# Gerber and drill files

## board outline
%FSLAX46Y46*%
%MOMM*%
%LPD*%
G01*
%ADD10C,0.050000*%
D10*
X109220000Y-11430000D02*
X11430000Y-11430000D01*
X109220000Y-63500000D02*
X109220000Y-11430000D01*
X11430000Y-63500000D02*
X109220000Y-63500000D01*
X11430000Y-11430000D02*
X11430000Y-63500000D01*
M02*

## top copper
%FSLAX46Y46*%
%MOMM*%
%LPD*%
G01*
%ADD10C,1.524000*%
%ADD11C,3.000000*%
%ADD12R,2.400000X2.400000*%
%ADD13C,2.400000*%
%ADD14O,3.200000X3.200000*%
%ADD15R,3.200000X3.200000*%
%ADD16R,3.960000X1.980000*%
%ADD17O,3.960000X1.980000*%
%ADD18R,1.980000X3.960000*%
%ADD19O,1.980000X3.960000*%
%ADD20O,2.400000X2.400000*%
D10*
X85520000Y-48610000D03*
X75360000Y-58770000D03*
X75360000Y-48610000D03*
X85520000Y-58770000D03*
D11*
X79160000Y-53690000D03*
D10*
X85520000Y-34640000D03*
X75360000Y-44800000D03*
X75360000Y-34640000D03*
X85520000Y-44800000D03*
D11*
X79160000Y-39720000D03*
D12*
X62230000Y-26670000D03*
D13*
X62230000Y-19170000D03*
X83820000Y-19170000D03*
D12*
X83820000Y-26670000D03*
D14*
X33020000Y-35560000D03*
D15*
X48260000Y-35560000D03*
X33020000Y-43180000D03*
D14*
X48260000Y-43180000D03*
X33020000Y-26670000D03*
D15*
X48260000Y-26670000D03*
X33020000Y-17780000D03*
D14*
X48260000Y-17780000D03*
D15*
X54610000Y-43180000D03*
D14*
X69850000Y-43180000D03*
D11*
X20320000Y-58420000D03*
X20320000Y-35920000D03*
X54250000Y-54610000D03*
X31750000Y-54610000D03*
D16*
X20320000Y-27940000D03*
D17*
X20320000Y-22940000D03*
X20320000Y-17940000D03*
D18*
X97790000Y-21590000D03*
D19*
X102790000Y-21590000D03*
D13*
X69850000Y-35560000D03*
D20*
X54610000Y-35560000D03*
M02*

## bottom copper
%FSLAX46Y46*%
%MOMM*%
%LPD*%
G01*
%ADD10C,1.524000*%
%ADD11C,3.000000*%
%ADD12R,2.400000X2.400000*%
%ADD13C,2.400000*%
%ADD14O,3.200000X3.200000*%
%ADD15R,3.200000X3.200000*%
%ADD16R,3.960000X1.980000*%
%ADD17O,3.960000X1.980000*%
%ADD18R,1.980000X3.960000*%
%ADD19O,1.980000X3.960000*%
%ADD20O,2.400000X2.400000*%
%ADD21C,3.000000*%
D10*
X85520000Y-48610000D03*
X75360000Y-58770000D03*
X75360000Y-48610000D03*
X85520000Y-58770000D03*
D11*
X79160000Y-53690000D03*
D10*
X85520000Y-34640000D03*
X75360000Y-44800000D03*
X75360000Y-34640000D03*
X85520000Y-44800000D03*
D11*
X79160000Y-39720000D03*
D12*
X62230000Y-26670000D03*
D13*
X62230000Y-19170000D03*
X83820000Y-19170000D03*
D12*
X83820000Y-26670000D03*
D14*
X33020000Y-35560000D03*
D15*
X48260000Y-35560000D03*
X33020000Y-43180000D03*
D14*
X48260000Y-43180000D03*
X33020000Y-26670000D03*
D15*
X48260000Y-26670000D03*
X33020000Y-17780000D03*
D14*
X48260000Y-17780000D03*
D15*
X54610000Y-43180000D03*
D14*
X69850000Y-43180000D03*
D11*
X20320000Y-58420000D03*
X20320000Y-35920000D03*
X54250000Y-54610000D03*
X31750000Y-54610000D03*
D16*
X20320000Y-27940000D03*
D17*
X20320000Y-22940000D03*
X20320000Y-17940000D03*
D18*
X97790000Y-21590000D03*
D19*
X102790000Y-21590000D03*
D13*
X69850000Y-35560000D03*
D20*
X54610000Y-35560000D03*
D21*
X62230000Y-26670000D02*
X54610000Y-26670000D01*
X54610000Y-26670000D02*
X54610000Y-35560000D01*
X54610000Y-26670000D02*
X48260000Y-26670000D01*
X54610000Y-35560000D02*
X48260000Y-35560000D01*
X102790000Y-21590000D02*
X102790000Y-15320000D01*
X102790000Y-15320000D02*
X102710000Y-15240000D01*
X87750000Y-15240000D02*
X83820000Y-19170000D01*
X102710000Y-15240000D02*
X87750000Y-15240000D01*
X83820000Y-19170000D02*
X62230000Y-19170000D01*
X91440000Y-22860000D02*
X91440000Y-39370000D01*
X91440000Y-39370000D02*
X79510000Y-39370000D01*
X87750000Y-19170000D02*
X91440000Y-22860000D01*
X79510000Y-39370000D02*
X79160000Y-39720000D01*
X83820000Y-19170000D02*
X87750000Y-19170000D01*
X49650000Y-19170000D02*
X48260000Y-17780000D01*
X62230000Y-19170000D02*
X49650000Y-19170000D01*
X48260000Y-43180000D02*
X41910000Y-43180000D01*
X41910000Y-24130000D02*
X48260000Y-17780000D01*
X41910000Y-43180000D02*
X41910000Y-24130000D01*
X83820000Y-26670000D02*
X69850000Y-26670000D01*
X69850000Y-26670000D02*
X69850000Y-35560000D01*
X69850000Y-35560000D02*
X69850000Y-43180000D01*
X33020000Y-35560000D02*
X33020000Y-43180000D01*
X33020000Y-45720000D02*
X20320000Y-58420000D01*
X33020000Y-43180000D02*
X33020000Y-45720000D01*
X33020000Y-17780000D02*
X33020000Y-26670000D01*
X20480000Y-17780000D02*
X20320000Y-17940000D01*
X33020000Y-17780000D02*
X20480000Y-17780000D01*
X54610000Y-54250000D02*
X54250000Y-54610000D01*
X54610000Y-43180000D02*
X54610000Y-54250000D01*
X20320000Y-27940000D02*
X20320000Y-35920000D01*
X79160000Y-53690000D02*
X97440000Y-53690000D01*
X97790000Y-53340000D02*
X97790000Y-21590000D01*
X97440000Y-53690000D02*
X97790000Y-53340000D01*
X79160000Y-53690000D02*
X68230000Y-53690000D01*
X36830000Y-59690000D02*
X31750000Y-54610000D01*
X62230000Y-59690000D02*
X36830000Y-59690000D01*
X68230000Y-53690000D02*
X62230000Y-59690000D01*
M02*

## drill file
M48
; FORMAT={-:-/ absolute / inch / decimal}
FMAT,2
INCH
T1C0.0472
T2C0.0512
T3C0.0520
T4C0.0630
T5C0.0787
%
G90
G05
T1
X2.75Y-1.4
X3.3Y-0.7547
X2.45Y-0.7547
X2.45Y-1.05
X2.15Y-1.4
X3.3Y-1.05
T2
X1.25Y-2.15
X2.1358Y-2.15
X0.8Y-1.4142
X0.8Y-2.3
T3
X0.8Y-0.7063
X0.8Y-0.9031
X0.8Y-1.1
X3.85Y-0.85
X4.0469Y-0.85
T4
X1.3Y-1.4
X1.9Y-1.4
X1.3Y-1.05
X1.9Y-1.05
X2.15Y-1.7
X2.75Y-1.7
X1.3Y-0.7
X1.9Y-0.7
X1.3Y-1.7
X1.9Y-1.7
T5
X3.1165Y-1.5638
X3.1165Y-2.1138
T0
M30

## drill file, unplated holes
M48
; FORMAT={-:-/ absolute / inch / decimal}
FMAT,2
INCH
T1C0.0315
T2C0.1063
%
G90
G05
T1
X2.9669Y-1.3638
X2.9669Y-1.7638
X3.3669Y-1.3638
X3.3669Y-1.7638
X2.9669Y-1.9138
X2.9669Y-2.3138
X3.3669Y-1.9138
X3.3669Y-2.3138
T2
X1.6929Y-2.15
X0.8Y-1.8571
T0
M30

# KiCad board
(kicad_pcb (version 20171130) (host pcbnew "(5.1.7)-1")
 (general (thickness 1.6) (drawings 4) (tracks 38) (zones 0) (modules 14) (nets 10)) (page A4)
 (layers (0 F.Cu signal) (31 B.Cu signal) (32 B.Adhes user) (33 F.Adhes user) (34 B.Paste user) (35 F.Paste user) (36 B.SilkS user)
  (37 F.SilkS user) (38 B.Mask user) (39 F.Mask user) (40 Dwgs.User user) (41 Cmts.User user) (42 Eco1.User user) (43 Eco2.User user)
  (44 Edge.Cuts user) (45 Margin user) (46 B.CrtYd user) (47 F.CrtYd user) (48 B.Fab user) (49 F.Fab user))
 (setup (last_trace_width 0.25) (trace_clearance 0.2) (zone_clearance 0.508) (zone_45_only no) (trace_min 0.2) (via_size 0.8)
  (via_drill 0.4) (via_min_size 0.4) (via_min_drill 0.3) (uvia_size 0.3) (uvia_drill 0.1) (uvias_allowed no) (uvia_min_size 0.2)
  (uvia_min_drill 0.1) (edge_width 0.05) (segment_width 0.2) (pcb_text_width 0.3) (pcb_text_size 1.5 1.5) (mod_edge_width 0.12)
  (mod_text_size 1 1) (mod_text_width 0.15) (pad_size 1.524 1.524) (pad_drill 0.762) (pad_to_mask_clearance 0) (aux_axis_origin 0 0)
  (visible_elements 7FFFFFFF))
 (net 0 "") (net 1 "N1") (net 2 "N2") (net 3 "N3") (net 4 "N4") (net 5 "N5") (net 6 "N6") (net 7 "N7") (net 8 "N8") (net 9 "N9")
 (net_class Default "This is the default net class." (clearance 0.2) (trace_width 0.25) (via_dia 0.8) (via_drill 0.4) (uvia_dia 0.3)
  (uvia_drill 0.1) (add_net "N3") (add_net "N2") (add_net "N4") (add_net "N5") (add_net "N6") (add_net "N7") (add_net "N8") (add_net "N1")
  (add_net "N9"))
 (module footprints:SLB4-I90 (layer F.Cu) (at 73.66 59.69)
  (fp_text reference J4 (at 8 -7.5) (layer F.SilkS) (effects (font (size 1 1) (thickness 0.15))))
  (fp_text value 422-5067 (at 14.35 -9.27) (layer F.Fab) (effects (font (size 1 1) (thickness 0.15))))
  (pad "" np_thru_hole circle (at 11.86 -11.08) (size 1.524 1.524) (drill 0.8) (layers *.Cu *.Mask))
  (pad "" np_thru_hole circle (at 1.7 -0.92) (size 1.524 1.524) (drill 0.8) (layers *.Cu *.Mask))
  (pad "" np_thru_hole circle (at 1.7 -11.08) (size 1.524 1.524) (drill 0.8) (layers *.Cu *.Mask))
  (pad "" np_thru_hole circle (at 11.86 -0.92) (size 1.524 1.524) (drill 0.8) (layers *.Cu *.Mask))
  (pad 1 thru_hole circle (at 5.5 -6) (size 3 3) (drill 2) (layers *.Cu *.Mask) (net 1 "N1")))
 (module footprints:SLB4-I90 (layer F.Cu) (at 73.66 45.72)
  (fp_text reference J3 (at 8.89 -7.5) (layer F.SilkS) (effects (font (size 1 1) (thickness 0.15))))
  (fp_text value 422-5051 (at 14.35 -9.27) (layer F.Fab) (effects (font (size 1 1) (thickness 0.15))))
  (pad "" np_thru_hole circle (at 11.86 -11.08) (size 1.524 1.524) (drill 0.8) (layers *.Cu *.Mask))
  (pad "" np_thru_hole circle (at 1.7 -0.92) (size 1.524 1.524) (drill 0.8) (layers *.Cu *.Mask))
  (pad "" np_thru_hole circle (at 1.7 -11.08) (size 1.524 1.524) (drill 0.8) (layers *.Cu *.Mask))
  (pad "" np_thru_hole circle (at 11.86 -0.92) (size 1.524 1.524) (drill 0.8) (layers *.Cu *.Mask))
  (pad 1 thru_hole circle (at 5.5 -6) (size 3 3) (drill 2) (layers *.Cu *.Mask) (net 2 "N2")))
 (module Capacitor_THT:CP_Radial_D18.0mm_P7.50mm (layer F.Cu) (at 62.23 26.67 90)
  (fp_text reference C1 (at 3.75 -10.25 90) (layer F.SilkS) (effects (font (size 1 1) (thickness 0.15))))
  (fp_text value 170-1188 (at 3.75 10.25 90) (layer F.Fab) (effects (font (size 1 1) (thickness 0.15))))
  (pad 1 thru_hole rect (at 0 0 90) (size 2.4 2.4) (drill 1.2) (layers *.Cu *.Mask) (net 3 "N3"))
  (pad 2 thru_hole circle (at 7.5 0 90) (size 2.4 2.4) (drill 1.2) (layers *.Cu *.Mask) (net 2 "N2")))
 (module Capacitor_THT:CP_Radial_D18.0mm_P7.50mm (layer F.Cu) (at 83.82 26.67 90)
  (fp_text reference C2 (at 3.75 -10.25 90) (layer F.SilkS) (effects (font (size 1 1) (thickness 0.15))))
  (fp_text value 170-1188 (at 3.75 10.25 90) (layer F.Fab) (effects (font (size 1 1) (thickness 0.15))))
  (pad 2 thru_hole circle (at 7.5 0 90) (size 2.4 2.4) (drill 1.2) (layers *.Cu *.Mask) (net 2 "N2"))
  (pad 1 thru_hole rect (at 0 0 90) (size 2.4 2.4) (drill 1.2) (layers *.Cu *.Mask) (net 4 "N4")))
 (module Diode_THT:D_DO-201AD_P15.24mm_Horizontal (layer F.Cu) (at 48.26 35.56 180)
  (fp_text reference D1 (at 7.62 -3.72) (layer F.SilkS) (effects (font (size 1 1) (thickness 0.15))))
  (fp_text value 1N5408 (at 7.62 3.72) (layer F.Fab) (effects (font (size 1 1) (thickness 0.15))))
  (pad 2 thru_hole oval (at 15.24 0 180) (size 3.2 3.2) (drill 1.6) (layers *.Cu *.Mask) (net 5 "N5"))
  (pad 1 thru_hole rect (at 0 0 180) (size 3.2 3.2) (drill 1.6) (layers *.Cu *.Mask) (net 3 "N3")))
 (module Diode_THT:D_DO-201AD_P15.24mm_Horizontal (layer F.Cu) (at 33.02 43.18)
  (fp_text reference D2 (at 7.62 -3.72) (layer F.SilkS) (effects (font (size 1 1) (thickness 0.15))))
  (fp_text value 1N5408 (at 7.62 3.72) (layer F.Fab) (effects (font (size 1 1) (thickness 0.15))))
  (pad 1 thru_hole rect (at 0 0) (size 3.2 3.2) (drill 1.6) (layers *.Cu *.Mask) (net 5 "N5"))
  (pad 2 thru_hole oval (at 15.24 0) (size 3.2 3.2) (drill 1.6) (layers *.Cu *.Mask) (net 2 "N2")))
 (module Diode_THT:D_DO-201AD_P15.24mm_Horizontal (layer F.Cu) (at 48.26 26.67 180)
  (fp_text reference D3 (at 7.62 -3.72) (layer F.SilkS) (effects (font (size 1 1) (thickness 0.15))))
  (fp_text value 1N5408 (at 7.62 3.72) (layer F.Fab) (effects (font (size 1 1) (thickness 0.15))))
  (pad 2 thru_hole oval (at 15.24 0 180) (size 3.2 3.2) (drill 1.6) (layers *.Cu *.Mask) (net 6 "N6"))
  (pad 1 thru_hole rect (at 0 0 180) (size 3.2 3.2) (drill 1.6) (layers *.Cu *.Mask) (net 3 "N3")))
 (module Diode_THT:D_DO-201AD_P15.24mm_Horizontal (layer F.Cu) (at 33.02 17.78)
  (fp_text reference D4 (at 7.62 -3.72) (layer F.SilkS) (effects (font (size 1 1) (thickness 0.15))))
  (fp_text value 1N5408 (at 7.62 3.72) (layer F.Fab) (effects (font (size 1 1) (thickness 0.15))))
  (pad 1 thru_hole rect (at 0 0) (size 3.2 3.2) (drill 1.6) (layers *.Cu *.Mask) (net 6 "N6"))
  (pad 2 thru_hole oval (at 15.24 0) (size 3.2 3.2) (drill 1.6) (layers *.Cu *.Mask) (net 2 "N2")))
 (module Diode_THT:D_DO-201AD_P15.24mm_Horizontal (layer F.Cu) (at 54.61 43.18)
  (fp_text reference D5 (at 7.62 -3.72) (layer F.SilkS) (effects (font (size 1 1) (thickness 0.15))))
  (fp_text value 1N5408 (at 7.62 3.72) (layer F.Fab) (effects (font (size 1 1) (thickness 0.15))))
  (pad 1 thru_hole rect (at 0 0) (size 3.2 3.2) (drill 1.6) (layers *.Cu *.Mask) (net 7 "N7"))
  (pad 2 thru_hole oval (at 15.24 0) (size 3.2 3.2) (drill 1.6) (layers *.Cu *.Mask) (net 4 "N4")))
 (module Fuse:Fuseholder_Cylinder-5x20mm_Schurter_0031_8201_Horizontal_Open (layer F.Cu) (at 20.32 58.42 90)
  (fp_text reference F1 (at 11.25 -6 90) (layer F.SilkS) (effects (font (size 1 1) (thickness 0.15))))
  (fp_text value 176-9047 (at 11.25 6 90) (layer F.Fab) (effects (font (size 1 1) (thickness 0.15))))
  (pad 1 thru_hole circle (at 0 0 90) (size 3 3) (drill 1.3) (layers *.Cu *.Mask) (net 5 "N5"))
  (pad 2 thru_hole circle (at 22.5 0 90) (size 3 3) (drill 1.3) (layers *.Cu *.Mask) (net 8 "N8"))
  (pad "" np_thru_hole circle (at 11.25 0 90) (size 2.7 2.7) (drill 2.7) (layers *.Cu *.Mask)))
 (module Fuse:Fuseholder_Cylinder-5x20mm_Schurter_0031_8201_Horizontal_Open (layer F.Cu) (at 31.75 54.61)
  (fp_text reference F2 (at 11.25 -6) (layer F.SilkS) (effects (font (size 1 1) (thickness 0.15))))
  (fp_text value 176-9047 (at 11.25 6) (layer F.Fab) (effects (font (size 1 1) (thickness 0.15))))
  (pad "" np_thru_hole circle (at 11.25 0) (size 2.7 2.7) (drill 2.7) (layers *.Cu *.Mask))
  (pad 2 thru_hole circle (at 22.5 0) (size 3 3) (drill 1.3) (layers *.Cu *.Mask) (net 7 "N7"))
  (pad 1 thru_hole circle (at 0 0) (size 3 3) (drill 1.3) (layers *.Cu *.Mask) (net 1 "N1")))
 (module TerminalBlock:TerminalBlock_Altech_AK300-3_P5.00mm (layer F.Cu) (at 20.32 27.94 90)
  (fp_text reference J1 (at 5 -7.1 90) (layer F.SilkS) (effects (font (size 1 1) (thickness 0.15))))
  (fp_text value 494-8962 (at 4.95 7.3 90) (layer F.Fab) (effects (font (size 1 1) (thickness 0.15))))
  (pad 1 thru_hole rect (at 0 0 90) (size 1.98 3.96) (drill 1.32) (layers *.Cu *.Mask) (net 8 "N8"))
  (pad 2 thru_hole oval (at 5 0 90) (size 1.98 3.96) (drill 1.32) (layers *.Cu *.Mask) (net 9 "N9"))
  (pad 3 thru_hole oval (at 10 0 90) (size 1.98 3.96) (drill 1.32) (layers *.Cu *.Mask) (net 6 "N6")))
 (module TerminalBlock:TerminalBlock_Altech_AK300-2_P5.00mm (layer F.Cu) (at 97.79 21.59)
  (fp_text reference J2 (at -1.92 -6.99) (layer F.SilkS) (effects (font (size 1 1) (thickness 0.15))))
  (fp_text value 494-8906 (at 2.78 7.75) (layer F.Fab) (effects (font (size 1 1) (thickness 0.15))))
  (pad 1 thru_hole rect (at 0 0) (size 1.98 3.96) (drill 1.32) (layers *.Cu *.Mask) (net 1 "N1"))
  (pad 2 thru_hole oval (at 5 0) (size 1.98 3.96) (drill 1.32) (layers *.Cu *.Mask) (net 2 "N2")))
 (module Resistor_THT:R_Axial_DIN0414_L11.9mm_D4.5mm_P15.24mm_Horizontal (layer F.Cu) (at 69.85 35.56 180)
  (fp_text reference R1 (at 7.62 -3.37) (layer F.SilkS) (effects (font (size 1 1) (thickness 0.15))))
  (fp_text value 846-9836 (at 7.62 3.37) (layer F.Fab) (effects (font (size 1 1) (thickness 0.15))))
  (pad 1 thru_hole circle (at 0 0 180) (size 2.4 2.4) (drill 1.2) (layers *.Cu *.Mask) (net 4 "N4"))
  (pad 2 thru_hole oval (at 15.24 0 180) (size 2.4 2.4) (drill 1.2) (layers *.Cu *.Mask) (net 3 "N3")))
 (gr_line (start 109.22 11.43) (end 11.43 11.43) (layer Edge.Cuts) (width 0.05))
 (gr_line (start 109.22 63.5) (end 109.22 11.43) (layer Edge.Cuts) (width 0.05))
 (gr_line (start 11.43 63.5) (end 109.22 63.5) (layer Edge.Cuts) (width 0.05))
 (gr_line (start 11.43 11.43) (end 11.43 63.5) (layer Edge.Cuts) (width 0.05))
 (segment (start 62.23 26.67) (end 54.61 26.67) (width 3) (layer B.Cu) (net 3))
 (segment (start 54.61 26.67) (end 54.61 35.56) (width 3) (layer B.Cu) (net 3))
 (segment (start 54.61 26.67) (end 48.26 26.67) (width 3) (layer B.Cu) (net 3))
 (segment (start 54.61 35.56) (end 48.26 35.56) (width 3) (layer B.Cu) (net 3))
 (segment (start 102.79 21.59) (end 102.79 15.32) (width 3) (layer B.Cu) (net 2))
 (segment (start 102.79 15.32) (end 102.71 15.24) (width 3) (layer B.Cu) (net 2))
 (segment (start 87.75 15.24) (end 83.82 19.17) (width 3) (layer B.Cu) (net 2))
 (segment (start 102.71 15.24) (end 87.75 15.24) (width 3) (layer B.Cu) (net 2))
 (segment (start 83.82 19.17) (end 62.23 19.17) (width 3) (layer B.Cu) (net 2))
 (segment (start 91.44 22.86) (end 91.44 39.37) (width 3) (layer B.Cu) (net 2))
 (segment (start 91.44 39.37) (end 79.51 39.37) (width 3) (layer B.Cu) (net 2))
 (segment (start 87.75 19.17) (end 91.44 22.86) (width 3) (layer B.Cu) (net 2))
 (segment (start 79.51 39.37) (end 79.16 39.72) (width 3) (layer B.Cu) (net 2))
 (segment (start 83.82 19.17) (end 87.75 19.17) (width 3) (layer B.Cu) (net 2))
 (segment (start 49.65 19.17) (end 48.26 17.78) (width 3) (layer B.Cu) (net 2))
 (segment (start 62.23 19.17) (end 49.65 19.17) (width 3) (layer B.Cu) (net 2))
 (segment (start 48.26 43.18) (end 41.91 43.18) (width 3) (layer B.Cu) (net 2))
 (segment (start 41.91 24.13) (end 48.26 17.78) (width 3) (layer B.Cu) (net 2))
 (segment (start 41.91 43.18) (end 41.91 24.13) (width 3) (layer B.Cu) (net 2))
 (segment (start 83.82 26.67) (end 69.85 26.67) (width 3) (layer B.Cu) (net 4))
 (segment (start 69.85 26.67) (end 69.85 35.56) (width 3) (layer B.Cu) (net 4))
 (segment (start 69.85 35.56) (end 69.85 43.18) (width 3) (layer B.Cu) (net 4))
 (segment (start 33.02 35.56) (end 33.02 43.18) (width 3) (layer B.Cu) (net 5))
 (segment (start 33.02 45.72) (end 20.32 58.42) (width 3) (layer B.Cu) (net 5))
 (segment (start 33.02 43.18) (end 33.02 45.72) (width 3) (layer B.Cu) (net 5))
 (segment (start 33.02 17.78) (end 33.02 26.67) (width 3) (layer B.Cu) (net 6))
 (segment (start 20.48 17.78) (end 20.32 17.94) (width 3) (layer B.Cu) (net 6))
 (segment (start 33.02 17.78) (end 20.48 17.78) (width 3) (layer B.Cu) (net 6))
 (segment (start 54.61 54.25) (end 54.25 54.61) (width 3) (layer B.Cu) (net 7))
 (segment (start 54.61 43.18) (end 54.61 54.25) (width 3) (layer B.Cu) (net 7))
 (segment (start 20.32 27.94) (end 20.32 35.92) (width 3) (layer B.Cu) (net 8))
 (segment (start 79.16 53.69) (end 97.44 53.69) (width 3) (layer B.Cu) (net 1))
 (segment (start 97.79 53.34) (end 97.79 21.59) (width 3) (layer B.Cu) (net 1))
 (segment (start 97.44 53.69) (end 97.79 53.34) (width 3) (layer B.Cu) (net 1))
 (segment (start 79.16 53.69) (end 68.23 53.69) (width 3) (layer B.Cu) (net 1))
 (segment (start 36.83 59.69) (end 31.75 54.61) (width 3) (layer B.Cu) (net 1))
 (segment (start 62.23 59.69) (end 36.83 59.69) (width 3) (layer B.Cu) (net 1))
 (segment (start 68.23 53.69) (end 62.23 59.69) (width 3) (layer B.Cu) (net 1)))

